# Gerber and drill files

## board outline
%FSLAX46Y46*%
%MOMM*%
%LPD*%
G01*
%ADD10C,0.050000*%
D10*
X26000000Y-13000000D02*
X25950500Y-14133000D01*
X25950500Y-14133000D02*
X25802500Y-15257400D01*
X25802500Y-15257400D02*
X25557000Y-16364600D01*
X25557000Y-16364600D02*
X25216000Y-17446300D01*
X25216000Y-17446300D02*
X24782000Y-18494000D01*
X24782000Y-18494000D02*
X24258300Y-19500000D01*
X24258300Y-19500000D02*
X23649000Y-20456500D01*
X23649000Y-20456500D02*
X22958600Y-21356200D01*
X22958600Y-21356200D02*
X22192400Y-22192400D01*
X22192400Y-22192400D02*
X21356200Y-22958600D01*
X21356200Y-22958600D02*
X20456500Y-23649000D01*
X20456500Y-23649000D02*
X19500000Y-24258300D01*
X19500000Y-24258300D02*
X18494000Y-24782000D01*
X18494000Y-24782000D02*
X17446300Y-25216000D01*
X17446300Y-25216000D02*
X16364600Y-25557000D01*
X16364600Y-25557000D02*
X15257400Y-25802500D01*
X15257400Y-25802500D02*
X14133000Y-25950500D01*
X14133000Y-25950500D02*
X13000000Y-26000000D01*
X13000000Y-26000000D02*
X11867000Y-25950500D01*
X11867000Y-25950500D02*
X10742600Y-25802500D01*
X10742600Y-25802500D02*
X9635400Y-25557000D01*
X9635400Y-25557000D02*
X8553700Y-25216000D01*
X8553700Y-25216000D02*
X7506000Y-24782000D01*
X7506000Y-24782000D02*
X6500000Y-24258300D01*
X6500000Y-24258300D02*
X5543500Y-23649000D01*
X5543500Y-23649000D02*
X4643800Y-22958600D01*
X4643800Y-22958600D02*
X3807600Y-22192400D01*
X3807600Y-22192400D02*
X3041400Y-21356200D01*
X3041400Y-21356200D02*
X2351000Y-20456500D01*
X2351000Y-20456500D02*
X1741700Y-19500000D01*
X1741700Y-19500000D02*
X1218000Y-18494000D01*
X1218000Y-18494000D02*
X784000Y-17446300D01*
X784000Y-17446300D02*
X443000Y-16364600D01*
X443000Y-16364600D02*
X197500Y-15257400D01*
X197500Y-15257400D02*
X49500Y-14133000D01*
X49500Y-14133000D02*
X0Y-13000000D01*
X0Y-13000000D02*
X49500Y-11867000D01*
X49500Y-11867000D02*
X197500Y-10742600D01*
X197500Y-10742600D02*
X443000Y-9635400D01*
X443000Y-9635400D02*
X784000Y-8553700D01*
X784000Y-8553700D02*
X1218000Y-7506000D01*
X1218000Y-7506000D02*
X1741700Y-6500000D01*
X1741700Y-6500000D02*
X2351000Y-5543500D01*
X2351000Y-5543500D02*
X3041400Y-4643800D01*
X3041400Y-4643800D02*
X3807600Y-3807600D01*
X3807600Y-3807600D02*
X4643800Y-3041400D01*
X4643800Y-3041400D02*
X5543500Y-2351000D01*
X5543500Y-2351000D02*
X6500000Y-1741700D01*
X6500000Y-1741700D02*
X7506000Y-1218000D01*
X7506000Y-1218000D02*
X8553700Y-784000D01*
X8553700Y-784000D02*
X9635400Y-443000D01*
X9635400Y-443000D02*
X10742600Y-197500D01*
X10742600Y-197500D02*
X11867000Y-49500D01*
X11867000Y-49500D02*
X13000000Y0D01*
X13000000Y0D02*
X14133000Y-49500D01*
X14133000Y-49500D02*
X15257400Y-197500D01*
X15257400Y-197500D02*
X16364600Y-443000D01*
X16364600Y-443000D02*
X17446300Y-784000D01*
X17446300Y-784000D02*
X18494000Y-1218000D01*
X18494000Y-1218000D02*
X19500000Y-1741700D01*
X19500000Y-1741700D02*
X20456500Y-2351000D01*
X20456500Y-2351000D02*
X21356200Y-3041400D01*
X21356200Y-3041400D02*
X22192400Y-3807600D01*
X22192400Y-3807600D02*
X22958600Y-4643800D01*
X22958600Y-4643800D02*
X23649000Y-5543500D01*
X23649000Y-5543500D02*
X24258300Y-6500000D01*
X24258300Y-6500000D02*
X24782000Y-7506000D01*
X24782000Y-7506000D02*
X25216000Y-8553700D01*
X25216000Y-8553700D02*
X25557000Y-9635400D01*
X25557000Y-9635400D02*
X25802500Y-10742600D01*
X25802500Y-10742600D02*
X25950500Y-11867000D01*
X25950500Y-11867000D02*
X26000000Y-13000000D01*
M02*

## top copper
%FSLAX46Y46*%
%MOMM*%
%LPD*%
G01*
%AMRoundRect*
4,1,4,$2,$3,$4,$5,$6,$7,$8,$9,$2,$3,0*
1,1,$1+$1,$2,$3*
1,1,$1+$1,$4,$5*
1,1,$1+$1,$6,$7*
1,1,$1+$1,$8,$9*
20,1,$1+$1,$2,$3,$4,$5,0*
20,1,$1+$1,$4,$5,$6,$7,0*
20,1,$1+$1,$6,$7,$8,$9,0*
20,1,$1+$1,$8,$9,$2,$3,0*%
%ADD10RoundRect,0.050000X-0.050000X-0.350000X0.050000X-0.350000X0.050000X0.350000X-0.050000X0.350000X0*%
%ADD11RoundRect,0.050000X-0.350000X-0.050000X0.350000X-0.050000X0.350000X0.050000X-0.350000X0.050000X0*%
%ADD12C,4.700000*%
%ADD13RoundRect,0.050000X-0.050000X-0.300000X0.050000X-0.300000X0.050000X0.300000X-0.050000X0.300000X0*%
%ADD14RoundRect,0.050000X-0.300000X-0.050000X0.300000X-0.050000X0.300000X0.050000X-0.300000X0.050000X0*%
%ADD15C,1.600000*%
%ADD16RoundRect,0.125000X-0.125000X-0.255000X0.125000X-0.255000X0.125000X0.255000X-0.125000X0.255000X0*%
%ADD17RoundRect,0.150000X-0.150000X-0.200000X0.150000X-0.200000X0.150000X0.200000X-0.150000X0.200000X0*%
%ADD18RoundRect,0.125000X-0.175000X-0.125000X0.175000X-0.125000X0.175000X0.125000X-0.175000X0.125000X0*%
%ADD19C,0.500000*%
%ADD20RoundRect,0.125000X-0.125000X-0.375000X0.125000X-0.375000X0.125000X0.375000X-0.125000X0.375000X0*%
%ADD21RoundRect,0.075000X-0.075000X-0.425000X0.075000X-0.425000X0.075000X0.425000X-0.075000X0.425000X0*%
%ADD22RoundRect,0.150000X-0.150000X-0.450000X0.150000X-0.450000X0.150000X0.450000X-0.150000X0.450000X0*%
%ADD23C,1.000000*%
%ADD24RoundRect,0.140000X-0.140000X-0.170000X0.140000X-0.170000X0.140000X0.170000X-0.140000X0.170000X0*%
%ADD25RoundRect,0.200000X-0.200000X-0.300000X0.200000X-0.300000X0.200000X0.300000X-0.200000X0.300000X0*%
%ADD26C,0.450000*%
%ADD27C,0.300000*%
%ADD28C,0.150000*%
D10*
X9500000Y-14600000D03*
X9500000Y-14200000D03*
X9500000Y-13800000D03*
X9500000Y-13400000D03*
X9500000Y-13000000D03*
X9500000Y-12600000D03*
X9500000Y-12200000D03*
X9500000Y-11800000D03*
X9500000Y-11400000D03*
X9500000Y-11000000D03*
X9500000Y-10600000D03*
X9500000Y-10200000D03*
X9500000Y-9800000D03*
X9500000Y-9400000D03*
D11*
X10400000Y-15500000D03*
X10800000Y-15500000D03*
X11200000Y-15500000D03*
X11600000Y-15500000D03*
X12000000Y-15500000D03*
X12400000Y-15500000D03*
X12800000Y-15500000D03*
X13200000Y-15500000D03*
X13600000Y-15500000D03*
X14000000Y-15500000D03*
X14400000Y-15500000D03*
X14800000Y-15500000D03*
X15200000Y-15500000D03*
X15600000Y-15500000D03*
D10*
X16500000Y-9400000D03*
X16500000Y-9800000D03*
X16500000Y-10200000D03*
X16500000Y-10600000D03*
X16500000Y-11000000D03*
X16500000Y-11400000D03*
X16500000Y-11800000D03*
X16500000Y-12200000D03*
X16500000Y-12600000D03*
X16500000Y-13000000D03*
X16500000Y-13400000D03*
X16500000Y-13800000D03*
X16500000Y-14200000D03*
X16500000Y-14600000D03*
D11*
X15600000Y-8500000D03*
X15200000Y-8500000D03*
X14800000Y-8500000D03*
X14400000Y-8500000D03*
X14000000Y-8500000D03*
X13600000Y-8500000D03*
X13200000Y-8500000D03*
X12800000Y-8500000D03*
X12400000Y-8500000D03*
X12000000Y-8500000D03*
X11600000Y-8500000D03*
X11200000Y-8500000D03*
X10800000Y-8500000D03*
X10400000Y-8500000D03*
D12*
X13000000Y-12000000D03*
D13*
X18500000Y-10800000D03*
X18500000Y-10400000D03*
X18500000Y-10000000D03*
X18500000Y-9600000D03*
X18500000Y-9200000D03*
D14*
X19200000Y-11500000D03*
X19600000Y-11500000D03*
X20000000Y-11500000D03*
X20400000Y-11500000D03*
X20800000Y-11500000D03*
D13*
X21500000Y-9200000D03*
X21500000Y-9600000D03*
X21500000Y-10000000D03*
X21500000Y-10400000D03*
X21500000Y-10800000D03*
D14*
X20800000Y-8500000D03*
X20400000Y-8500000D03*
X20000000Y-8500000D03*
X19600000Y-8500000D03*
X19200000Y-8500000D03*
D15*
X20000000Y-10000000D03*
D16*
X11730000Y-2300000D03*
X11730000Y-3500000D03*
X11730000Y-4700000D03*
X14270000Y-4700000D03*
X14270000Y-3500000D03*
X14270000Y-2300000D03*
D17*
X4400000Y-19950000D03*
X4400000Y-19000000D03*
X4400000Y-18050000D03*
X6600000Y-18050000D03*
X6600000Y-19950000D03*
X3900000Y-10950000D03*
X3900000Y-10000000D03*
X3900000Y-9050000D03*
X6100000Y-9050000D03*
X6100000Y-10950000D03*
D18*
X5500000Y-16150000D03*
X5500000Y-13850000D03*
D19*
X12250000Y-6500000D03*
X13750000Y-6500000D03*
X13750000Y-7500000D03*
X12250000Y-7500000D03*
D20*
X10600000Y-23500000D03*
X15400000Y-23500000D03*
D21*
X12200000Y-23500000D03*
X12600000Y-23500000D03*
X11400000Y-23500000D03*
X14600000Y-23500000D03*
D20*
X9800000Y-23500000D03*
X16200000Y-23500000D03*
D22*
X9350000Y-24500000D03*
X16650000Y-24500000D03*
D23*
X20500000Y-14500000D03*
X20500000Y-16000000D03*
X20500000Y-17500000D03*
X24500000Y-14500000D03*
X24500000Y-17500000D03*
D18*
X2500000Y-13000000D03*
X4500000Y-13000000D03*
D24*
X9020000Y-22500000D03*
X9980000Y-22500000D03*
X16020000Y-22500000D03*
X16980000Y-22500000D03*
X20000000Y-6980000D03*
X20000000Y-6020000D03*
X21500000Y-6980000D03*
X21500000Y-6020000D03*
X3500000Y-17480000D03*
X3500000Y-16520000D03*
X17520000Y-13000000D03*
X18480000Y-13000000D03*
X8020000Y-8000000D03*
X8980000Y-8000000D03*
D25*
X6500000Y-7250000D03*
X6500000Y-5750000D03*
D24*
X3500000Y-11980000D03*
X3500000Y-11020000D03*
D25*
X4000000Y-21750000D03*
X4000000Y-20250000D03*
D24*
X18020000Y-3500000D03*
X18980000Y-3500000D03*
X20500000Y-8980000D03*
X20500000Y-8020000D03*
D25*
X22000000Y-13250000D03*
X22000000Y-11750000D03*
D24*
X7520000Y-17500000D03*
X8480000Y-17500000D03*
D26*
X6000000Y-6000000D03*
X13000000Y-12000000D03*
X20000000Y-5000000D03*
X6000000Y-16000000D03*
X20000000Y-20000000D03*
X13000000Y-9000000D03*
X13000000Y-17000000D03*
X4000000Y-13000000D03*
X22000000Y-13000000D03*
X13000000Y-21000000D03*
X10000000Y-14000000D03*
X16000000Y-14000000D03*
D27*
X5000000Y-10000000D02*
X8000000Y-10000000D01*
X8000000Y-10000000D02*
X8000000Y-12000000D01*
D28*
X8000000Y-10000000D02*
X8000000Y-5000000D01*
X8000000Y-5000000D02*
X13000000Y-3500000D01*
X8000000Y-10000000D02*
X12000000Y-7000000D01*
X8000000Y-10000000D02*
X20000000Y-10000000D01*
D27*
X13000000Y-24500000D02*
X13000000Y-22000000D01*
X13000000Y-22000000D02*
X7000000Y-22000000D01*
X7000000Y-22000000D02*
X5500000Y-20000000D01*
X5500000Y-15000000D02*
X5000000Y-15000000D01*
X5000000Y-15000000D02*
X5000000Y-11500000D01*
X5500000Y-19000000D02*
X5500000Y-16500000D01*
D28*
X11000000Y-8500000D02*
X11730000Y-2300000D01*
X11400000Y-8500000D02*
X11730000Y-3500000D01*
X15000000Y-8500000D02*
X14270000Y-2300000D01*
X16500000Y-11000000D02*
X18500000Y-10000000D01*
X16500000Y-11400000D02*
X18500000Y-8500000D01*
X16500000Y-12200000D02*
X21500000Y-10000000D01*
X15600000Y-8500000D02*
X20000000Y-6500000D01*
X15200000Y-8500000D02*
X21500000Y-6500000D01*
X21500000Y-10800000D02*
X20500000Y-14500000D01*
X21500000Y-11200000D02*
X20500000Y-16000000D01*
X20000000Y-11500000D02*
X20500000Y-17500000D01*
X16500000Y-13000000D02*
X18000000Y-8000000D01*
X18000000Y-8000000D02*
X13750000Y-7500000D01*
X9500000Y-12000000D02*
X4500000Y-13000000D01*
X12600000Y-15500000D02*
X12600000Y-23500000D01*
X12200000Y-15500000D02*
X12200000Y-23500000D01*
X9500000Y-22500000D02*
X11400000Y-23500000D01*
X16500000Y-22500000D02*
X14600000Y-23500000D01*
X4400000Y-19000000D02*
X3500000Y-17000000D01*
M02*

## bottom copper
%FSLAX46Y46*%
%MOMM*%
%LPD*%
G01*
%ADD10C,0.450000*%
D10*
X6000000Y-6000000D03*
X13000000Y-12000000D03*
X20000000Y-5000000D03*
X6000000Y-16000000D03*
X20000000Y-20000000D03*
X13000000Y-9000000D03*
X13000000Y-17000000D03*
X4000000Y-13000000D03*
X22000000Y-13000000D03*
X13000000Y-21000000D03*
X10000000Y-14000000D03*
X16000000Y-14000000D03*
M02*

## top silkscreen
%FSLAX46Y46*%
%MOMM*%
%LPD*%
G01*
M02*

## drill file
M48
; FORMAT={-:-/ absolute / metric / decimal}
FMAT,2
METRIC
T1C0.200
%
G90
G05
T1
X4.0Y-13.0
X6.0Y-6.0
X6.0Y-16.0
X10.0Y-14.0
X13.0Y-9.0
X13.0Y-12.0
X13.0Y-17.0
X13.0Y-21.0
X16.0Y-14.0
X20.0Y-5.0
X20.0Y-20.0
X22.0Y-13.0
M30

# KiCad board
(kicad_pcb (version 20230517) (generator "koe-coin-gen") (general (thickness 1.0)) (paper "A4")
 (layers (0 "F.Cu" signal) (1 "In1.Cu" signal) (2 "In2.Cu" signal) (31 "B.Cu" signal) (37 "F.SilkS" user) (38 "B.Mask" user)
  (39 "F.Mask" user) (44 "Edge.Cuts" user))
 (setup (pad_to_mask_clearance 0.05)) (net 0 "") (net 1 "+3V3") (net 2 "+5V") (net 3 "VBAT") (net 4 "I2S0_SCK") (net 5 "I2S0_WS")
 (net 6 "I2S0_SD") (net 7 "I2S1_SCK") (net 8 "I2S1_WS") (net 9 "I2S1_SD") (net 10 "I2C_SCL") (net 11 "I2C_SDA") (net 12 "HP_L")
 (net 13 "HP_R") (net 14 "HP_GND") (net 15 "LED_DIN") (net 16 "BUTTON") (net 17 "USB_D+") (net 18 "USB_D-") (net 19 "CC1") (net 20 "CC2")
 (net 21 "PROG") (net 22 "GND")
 (gr_line (start 26.0000 13.0000) (end 25.9505 14.1330) (layer "Edge.Cuts") (width 0.05))
 (gr_line (start 25.9505 14.1330) (end 25.8025 15.2574) (layer "Edge.Cuts") (width 0.05))
 (gr_line (start 25.8025 15.2574) (end 25.5570 16.3646) (layer "Edge.Cuts") (width 0.05))
 (gr_line (start 25.5570 16.3646) (end 25.2160 17.4463) (layer "Edge.Cuts") (width 0.05))
 (gr_line (start 25.2160 17.4463) (end 24.7820 18.4940) (layer "Edge.Cuts") (width 0.05))
 (gr_line (start 24.7820 18.4940) (end 24.2583 19.5000) (layer "Edge.Cuts") (width 0.05))
 (gr_line (start 24.2583 19.5000) (end 23.6490 20.4565) (layer "Edge.Cuts") (width 0.05))
 (gr_line (start 23.6490 20.4565) (end 22.9586 21.3562) (layer "Edge.Cuts") (width 0.05))
 (gr_line (start 22.9586 21.3562) (end 22.1924 22.1924) (layer "Edge.Cuts") (width 0.05))
 (gr_line (start 22.1924 22.1924) (end 21.3562 22.9586) (layer "Edge.Cuts") (width 0.05))
 (gr_line (start 21.3562 22.9586) (end 20.4565 23.6490) (layer "Edge.Cuts") (width 0.05))
 (gr_line (start 20.4565 23.6490) (end 19.5000 24.2583) (layer "Edge.Cuts") (width 0.05))
 (gr_line (start 19.5000 24.2583) (end 18.4940 24.7820) (layer "Edge.Cuts") (width 0.05))
 (gr_line (start 18.4940 24.7820) (end 17.4463 25.2160) (layer "Edge.Cuts") (width 0.05))
 (gr_line (start 17.4463 25.2160) (end 16.3646 25.5570) (layer "Edge.Cuts") (width 0.05))
 (gr_line (start 16.3646 25.5570) (end 15.2574 25.8025) (layer "Edge.Cuts") (width 0.05))
 (gr_line (start 15.2574 25.8025) (end 14.1330 25.9505) (layer "Edge.Cuts") (width 0.05))
 (gr_line (start 14.1330 25.9505) (end 13.0000 26.0000) (layer "Edge.Cuts") (width 0.05))
 (gr_line (start 13.0000 26.0000) (end 11.8670 25.9505) (layer "Edge.Cuts") (width 0.05))
 (gr_line (start 11.8670 25.9505) (end 10.7426 25.8025) (layer "Edge.Cuts") (width 0.05))
 (gr_line (start 10.7426 25.8025) (end 9.6354 25.5570) (layer "Edge.Cuts") (width 0.05))
 (gr_line (start 9.6354 25.5570) (end 8.5537 25.2160) (layer "Edge.Cuts") (width 0.05))
 (gr_line (start 8.5537 25.2160) (end 7.5060 24.7820) (layer "Edge.Cuts") (width 0.05))
 (gr_line (start 7.5060 24.7820) (end 6.5000 24.2583) (layer "Edge.Cuts") (width 0.05))
 (gr_line (start 6.5000 24.2583) (end 5.5435 23.6490) (layer "Edge.Cuts") (width 0.05))
 (gr_line (start 5.5435 23.6490) (end 4.6438 22.9586) (layer "Edge.Cuts") (width 0.05))
 (gr_line (start 4.6438 22.9586) (end 3.8076 22.1924) (layer "Edge.Cuts") (width 0.05))
 (gr_line (start 3.8076 22.1924) (end 3.0414 21.3562) (layer "Edge.Cuts") (width 0.05))
 (gr_line (start 3.0414 21.3562) (end 2.3510 20.4565) (layer "Edge.Cuts") (width 0.05))
 (gr_line (start 2.3510 20.4565) (end 1.7417 19.5000) (layer "Edge.Cuts") (width 0.05))
 (gr_line (start 1.7417 19.5000) (end 1.2180 18.4940) (layer "Edge.Cuts") (width 0.05))
 (gr_line (start 1.2180 18.4940) (end 0.7840 17.4463) (layer "Edge.Cuts") (width 0.05))
 (gr_line (start 0.7840 17.4463) (end 0.4430 16.3646) (layer "Edge.Cuts") (width 0.05))
 (gr_line (start 0.4430 16.3646) (end 0.1975 15.2574) (layer "Edge.Cuts") (width 0.05))
 (gr_line (start 0.1975 15.2574) (end 0.0495 14.1330) (layer "Edge.Cuts") (width 0.05))
 (gr_line (start 0.0495 14.1330) (end 0.0000 13.0000) (layer "Edge.Cuts") (width 0.05))
 (gr_line (start 0.0000 13.0000) (end 0.0495 11.8670) (layer "Edge.Cuts") (width 0.05))
 (gr_line (start 0.0495 11.8670) (end 0.1975 10.7426) (layer "Edge.Cuts") (width 0.05))
 (gr_line (start 0.1975 10.7426) (end 0.4430 9.6354) (layer "Edge.Cuts") (width 0.05))
 (gr_line (start 0.4430 9.6354) (end 0.7840 8.5537) (layer "Edge.Cuts") (width 0.05))
 (gr_line (start 0.7840 8.5537) (end 1.2180 7.5060) (layer "Edge.Cuts") (width 0.05))
 (gr_line (start 1.2180 7.5060) (end 1.7417 6.5000) (layer "Edge.Cuts") (width 0.05))
 (gr_line (start 1.7417 6.5000) (end 2.3510 5.5435) (layer "Edge.Cuts") (width 0.05))
 (gr_line (start 2.3510 5.5435) (end 3.0414 4.6438) (layer "Edge.Cuts") (width 0.05))
 (gr_line (start 3.0414 4.6438) (end 3.8076 3.8076) (layer "Edge.Cuts") (width 0.05))
 (gr_line (start 3.8076 3.8076) (end 4.6438 3.0414) (layer "Edge.Cuts") (width 0.05))
 (gr_line (start 4.6438 3.0414) (end 5.5435 2.3510) (layer "Edge.Cuts") (width 0.05))
 (gr_line (start 5.5435 2.3510) (end 6.5000 1.7417) (layer "Edge.Cuts") (width 0.05))
 (gr_line (start 6.5000 1.7417) (end 7.5060 1.2180) (layer "Edge.Cuts") (width 0.05))
 (gr_line (start 7.5060 1.2180) (end 8.5537 0.7840) (layer "Edge.Cuts") (width 0.05))
 (gr_line (start 8.5537 0.7840) (end 9.6354 0.4430) (layer "Edge.Cuts") (width 0.05))
 (gr_line (start 9.6354 0.4430) (end 10.7426 0.1975) (layer "Edge.Cuts") (width 0.05))
 (gr_line (start 10.7426 0.1975) (end 11.8670 0.0495) (layer "Edge.Cuts") (width 0.05))
 (gr_line (start 11.8670 0.0495) (end 13.0000 0.0000) (layer "Edge.Cuts") (width 0.05))
 (gr_line (start 13.0000 0.0000) (end 14.1330 0.0495) (layer "Edge.Cuts") (width 0.05))
 (gr_line (start 14.1330 0.0495) (end 15.2574 0.1975) (layer "Edge.Cuts") (width 0.05))
 (gr_line (start 15.2574 0.1975) (end 16.3646 0.4430) (layer "Edge.Cuts") (width 0.05))
 (gr_line (start 16.3646 0.4430) (end 17.4463 0.7840) (layer "Edge.Cuts") (width 0.05))
 (gr_line (start 17.4463 0.7840) (end 18.4940 1.2180) (layer "Edge.Cuts") (width 0.05))
 (gr_line (start 18.4940 1.2180) (end 19.5000 1.7417) (layer "Edge.Cuts") (width 0.05))
 (gr_line (start 19.5000 1.7417) (end 20.4565 2.3510) (layer "Edge.Cuts") (width 0.05))
 (gr_line (start 20.4565 2.3510) (end 21.3562 3.0414) (layer "Edge.Cuts") (width 0.05))
 (gr_line (start 21.3562 3.0414) (end 22.1924 3.8076) (layer "Edge.Cuts") (width 0.05))
 (gr_line (start 22.1924 3.8076) (end 22.9586 4.6438) (layer "Edge.Cuts") (width 0.05))
 (gr_line (start 22.9586 4.6438) (end 23.6490 5.5435) (layer "Edge.Cuts") (width 0.05))
 (gr_line (start 23.6490 5.5435) (end 24.2583 6.5000) (layer "Edge.Cuts") (width 0.05))
 (gr_line (start 24.2583 6.5000) (end 24.7820 7.5060) (layer "Edge.Cuts") (width 0.05))
 (gr_line (start 24.7820 7.5060) (end 25.2160 8.5537) (layer "Edge.Cuts") (width 0.05))
 (gr_line (start 25.2160 8.5537) (end 25.5570 9.6354) (layer "Edge.Cuts") (width 0.05))
 (gr_line (start 25.5570 9.6354) (end 25.8025 10.7426) (layer "Edge.Cuts") (width 0.05))
 (gr_line (start 25.8025 10.7426) (end 25.9505 11.8670) (layer "Edge.Cuts") (width 0.05))
 (gr_line (start 25.9505 11.8670) (end 26.0000 13.0000) (layer "Edge.Cuts") (width 0.05))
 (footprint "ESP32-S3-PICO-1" (at 13.0 12.0 0) (layer "F.Cu") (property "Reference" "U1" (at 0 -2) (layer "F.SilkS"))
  (pad "1" smd roundrect (at -3.5 2.6) (size 0.2 0.8) (layers "F.Cu" "F.Paste" "F.Mask") (roundrect_rratio 0.25))
  (pad "2" smd roundrect (at -3.5 2.2) (size 0.2 0.8) (layers "F.Cu" "F.Paste" "F.Mask") (roundrect_rratio 0.25))
  (pad "3" smd roundrect (at -3.5 1.8) (size 0.2 0.8) (layers "F.Cu" "F.Paste" "F.Mask") (roundrect_rratio 0.25))
  (pad "4" smd roundrect (at -3.5 1.4) (size 0.2 0.8) (layers "F.Cu" "F.Paste" "F.Mask") (roundrect_rratio 0.25))
  (pad "5" smd roundrect (at -3.5 1.0) (size 0.2 0.8) (layers "F.Cu" "F.Paste" "F.Mask") (roundrect_rratio 0.25))
  (pad "6" smd roundrect (at -3.5 0.6000000000000001) (size 0.2 0.8) (layers "F.Cu" "F.Paste" "F.Mask") (roundrect_rratio 0.25))
  (pad "7" smd roundrect (at -3.5 0.19999999999999973) (size 0.2 0.8) (layers "F.Cu" "F.Paste" "F.Mask") (roundrect_rratio 0.25))
  (pad "8" smd roundrect (at -3.5 -0.20000000000000018) (size 0.2 0.8) (layers "F.Cu" "F.Paste" "F.Mask") (roundrect_rratio 0.25))
  (pad "9" smd roundrect (at -3.5 -0.6000000000000001) (size 0.2 0.8) (layers "F.Cu" "F.Paste" "F.Mask") (roundrect_rratio 0.25))
  (pad "10" smd roundrect (at -3.5 -1.0) (size 0.2 0.8) (layers "F.Cu" "F.Paste" "F.Mask") (roundrect_rratio 0.25))
  (pad "11" smd roundrect (at -3.5 -1.4) (size 0.2 0.8) (layers "F.Cu" "F.Paste" "F.Mask") (roundrect_rratio 0.25))
  (pad "12" smd roundrect (at -3.5 -1.8000000000000003) (size 0.2 0.8) (layers "F.Cu" "F.Paste" "F.Mask") (roundrect_rratio 0.25))
  (pad "13" smd roundrect (at -3.5 -2.2000000000000006) (size 0.2 0.8) (layers "F.Cu" "F.Paste" "F.Mask") (roundrect_rratio 0.25))
  (pad "14" smd roundrect (at -3.5 -2.6) (size 0.2 0.8) (layers "F.Cu" "F.Paste" "F.Mask") (roundrect_rratio 0.25))
  (pad "15" smd roundrect (at -2.6 3.5) (size 0.8 0.2) (layers "F.Cu" "F.Paste" "F.Mask") (roundrect_rratio 0.25))
  (pad "16" smd roundrect (at -2.2 3.5) (size 0.8 0.2) (layers "F.Cu" "F.Paste" "F.Mask") (roundrect_rratio 0.25))
  (pad "17" smd roundrect (at -1.8 3.5) (size 0.8 0.2) (layers "F.Cu" "F.Paste" "F.Mask") (roundrect_rratio 0.25))
  (pad "18" smd roundrect (at -1.4 3.5) (size 0.8 0.2) (layers "F.Cu" "F.Paste" "F.Mask") (roundrect_rratio 0.25))
  (pad "19" smd roundrect (at -1.0 3.5) (size 0.8 0.2) (layers "F.Cu" "F.Paste" "F.Mask") (roundrect_rratio 0.25))
  (pad "20" smd roundrect (at -0.6000000000000001 3.5) (size 0.8 0.2) (layers "F.Cu" "F.Paste" "F.Mask") (roundrect_rratio 0.25))
  (pad "21" smd roundrect (at -0.19999999999999973 3.5) (size 0.8 0.2) (layers "F.Cu" "F.Paste" "F.Mask") (roundrect_rratio 0.25))
  (pad "22" smd roundrect (at 0.20000000000000018 3.5) (size 0.8 0.2) (layers "F.Cu" "F.Paste" "F.Mask") (roundrect_rratio 0.25))
  (pad "23" smd roundrect (at 0.6000000000000001 3.5) (size 0.8 0.2) (layers "F.Cu" "F.Paste" "F.Mask") (roundrect_rratio 0.25))
  (pad "24" smd roundrect (at 1.0 3.5) (size 0.8 0.2) (layers "F.Cu" "F.Paste" "F.Mask") (roundrect_rratio 0.25))
  (pad "25" smd roundrect (at 1.4 3.5) (size 0.8 0.2) (layers "F.Cu" "F.Paste" "F.Mask") (roundrect_rratio 0.25))
  (pad "26" smd roundrect (at 1.8000000000000003 3.5) (size 0.8 0.2) (layers "F.Cu" "F.Paste" "F.Mask") (roundrect_rratio 0.25))
  (pad "27" smd roundrect (at 2.2000000000000006 3.5) (size 0.8 0.2) (layers "F.Cu" "F.Paste" "F.Mask") (roundrect_rratio 0.25))
  (pad "28" smd roundrect (at 2.6 3.5) (size 0.8 0.2) (layers "F.Cu" "F.Paste" "F.Mask") (roundrect_rratio 0.25))
  (pad "29" smd roundrect (at 3.5 -2.6) (size 0.2 0.8) (layers "F.Cu" "F.Paste" "F.Mask") (roundrect_rratio 0.25))
  (pad "30" smd roundrect (at 3.5 -2.2) (size 0.2 0.8) (layers "F.Cu" "F.Paste" "F.Mask") (roundrect_rratio 0.25))
  (pad "31" smd roundrect (at 3.5 -1.8) (size 0.2 0.8) (layers "F.Cu" "F.Paste" "F.Mask") (roundrect_rratio 0.25))
  (pad "32" smd roundrect (at 3.5 -1.4) (size 0.2 0.8) (layers "F.Cu" "F.Paste" "F.Mask") (roundrect_rratio 0.25))
  (pad "33" smd roundrect (at 3.5 -1.0) (size 0.2 0.8) (layers "F.Cu" "F.Paste" "F.Mask") (roundrect_rratio 0.25))
  (pad "34" smd roundrect (at 3.5 -0.6000000000000001) (size 0.2 0.8) (layers "F.Cu" "F.Paste" "F.Mask") (roundrect_rratio 0.25))
  (pad "35" smd roundrect (at 3.5 -0.19999999999999973) (size 0.2 0.8) (layers "F.Cu" "F.Paste" "F.Mask") (roundrect_rratio 0.25))
  (pad "36" smd roundrect (at 3.5 0.20000000000000018) (size 0.2 0.8) (layers "F.Cu" "F.Paste" "F.Mask") (roundrect_rratio 0.25))
  (pad "37" smd roundrect (at 3.5 0.6000000000000001) (size 0.2 0.8) (layers "F.Cu" "F.Paste" "F.Mask") (roundrect_rratio 0.25))
  (pad "38" smd roundrect (at 3.5 1.0) (size 0.2 0.8) (layers "F.Cu" "F.Paste" "F.Mask") (roundrect_rratio 0.25))
  (pad "39" smd roundrect (at 3.5 1.4) (size 0.2 0.8) (layers "F.Cu" "F.Paste" "F.Mask") (roundrect_rratio 0.25))
  (pad "40" smd roundrect (at 3.5 1.8000000000000003) (size 0.2 0.8) (layers "F.Cu" "F.Paste" "F.Mask") (roundrect_rratio 0.25))
  (pad "41" smd roundrect (at 3.5 2.2000000000000006) (size 0.2 0.8) (layers "F.Cu" "F.Paste" "F.Mask") (roundrect_rratio 0.25))
  (pad "42" smd roundrect (at 3.5 2.6) (size 0.2 0.8) (layers "F.Cu" "F.Paste" "F.Mask") (roundrect_rratio 0.25))
  (pad "43" smd roundrect (at 2.6 -3.5) (size 0.8 0.2) (layers "F.Cu" "F.Paste" "F.Mask") (roundrect_rratio 0.25))
  (pad "44" smd roundrect (at 2.2 -3.5) (size 0.8 0.2) (layers "F.Cu" "F.Paste" "F.Mask") (roundrect_rratio 0.25))
  (pad "45" smd roundrect (at 1.8 -3.5) (size 0.8 0.2) (layers "F.Cu" "F.Paste" "F.Mask") (roundrect_rratio 0.25))
  (pad "46" smd roundrect (at 1.4 -3.5) (size 0.8 0.2) (layers "F.Cu" "F.Paste" "F.Mask") (roundrect_rratio 0.25))
  (pad "47" smd roundrect (at 1.0 -3.5) (size 0.8 0.2) (layers "F.Cu" "F.Paste" "F.Mask") (roundrect_rratio 0.25))
  (pad "48" smd roundrect (at 0.6000000000000001 -3.5) (size 0.8 0.2) (layers "F.Cu" "F.Paste" "F.Mask") (roundrect_rratio 0.25))
  (pad "49" smd roundrect (at 0.19999999999999973 -3.5) (size 0.8 0.2) (layers "F.Cu" "F.Paste" "F.Mask") (roundrect_rratio 0.25))
  (pad "50" smd roundrect (at -0.20000000000000018 -3.5) (size 0.8 0.2) (layers "F.Cu" "F.Paste" "F.Mask") (roundrect_rratio 0.25))
  (pad "51" smd roundrect (at -0.6000000000000001 -3.5) (size 0.8 0.2) (layers "F.Cu" "F.Paste" "F.Mask") (roundrect_rratio 0.25))
  (pad "52" smd roundrect (at -1.0 -3.5) (size 0.8 0.2) (layers "F.Cu" "F.Paste" "F.Mask") (roundrect_rratio 0.25))
  (pad "53" smd roundrect (at -1.4 -3.5) (size 0.8 0.2) (layers "F.Cu" "F.Paste" "F.Mask") (roundrect_rratio 0.25))
  (pad "54" smd roundrect (at -1.8000000000000003 -3.5) (size 0.8 0.2) (layers "F.Cu" "F.Paste" "F.Mask") (roundrect_rratio 0.25))
  (pad "55" smd roundrect (at -2.2000000000000006 -3.5) (size 0.8 0.2) (layers "F.Cu" "F.Paste" "F.Mask") (roundrect_rratio 0.25))
  (pad "56" smd roundrect (at -2.6 -3.5) (size 0.8 0.2) (layers "F.Cu" "F.Paste" "F.Mask") (roundrect_rratio 0.25))
  (pad "57" smd circle (at 0.0 0.0) (size 4.7 4.7) (layers "F.Cu" "F.Paste" "F.Mask") (roundrect_rratio 0.25)))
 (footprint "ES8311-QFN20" (at 20.0 10.0 0) (layer "F.Cu") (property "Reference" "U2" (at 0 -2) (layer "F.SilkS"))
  (pad "1" smd roundrect (at -1.5 0.8) (size 0.2 0.7) (layers "F.Cu" "F.Paste" "F.Mask") (roundrect_rratio 0.25))
  (pad "2" smd roundrect (at -1.5 0.4) (size 0.2 0.7) (layers "F.Cu" "F.Paste" "F.Mask") (roundrect_rratio 0.25))
  (pad "3" smd roundrect (at -1.5 0.0) (size 0.2 0.7) (layers "F.Cu" "F.Paste" "F.Mask") (roundrect_rratio 0.25))
  (pad "4" smd roundrect (at -1.5 -0.40000000000000013) (size 0.2 0.7) (layers "F.Cu" "F.Paste" "F.Mask") (roundrect_rratio 0.25))
  (pad "5" smd roundrect (at -1.5 -0.8) (size 0.2 0.7) (layers "F.Cu" "F.Paste" "F.Mask") (roundrect_rratio 0.25))
  (pad "6" smd roundrect (at -0.8 1.5) (size 0.7 0.2) (layers "F.Cu" "F.Paste" "F.Mask") (roundrect_rratio 0.25))
  (pad "7" smd roundrect (at -0.4 1.5) (size 0.7 0.2) (layers "F.Cu" "F.Paste" "F.Mask") (roundrect_rratio 0.25))
  (pad "8" smd roundrect (at 0.0 1.5) (size 0.7 0.2) (layers "F.Cu" "F.Paste" "F.Mask") (roundrect_rratio 0.25))
  (pad "9" smd roundrect (at 0.40000000000000013 1.5) (size 0.7 0.2) (layers "F.Cu" "F.Paste" "F.Mask") (roundrect_rratio 0.25))
  (pad "10" smd roundrect (at 0.8 1.5) (size 0.7 0.2) (layers "F.Cu" "F.Paste" "F.Mask") (roundrect_rratio 0.25))
  (pad "11" smd roundrect (at 1.5 -0.8) (size 0.2 0.7) (layers "F.Cu" "F.Paste" "F.Mask") (roundrect_rratio 0.25))
  (pad "12" smd roundrect (at 1.5 -0.4) (size 0.2 0.7) (layers "F.Cu" "F.Paste" "F.Mask") (roundrect_rratio 0.25))
  (pad "13" smd roundrect (at 1.5 0.0) (size 0.2 0.7) (layers "F.Cu" "F.Paste" "F.Mask") (roundrect_rratio 0.25))
  (pad "14" smd roundrect (at 1.5 0.40000000000000013) (size 0.2 0.7) (layers "F.Cu" "F.Paste" "F.Mask") (roundrect_rratio 0.25))
  (pad "15" smd roundrect (at 1.5 0.8) (size 0.2 0.7) (layers "F.Cu" "F.Paste" "F.Mask") (roundrect_rratio 0.25))
  (pad "16" smd roundrect (at 0.8 -1.5) (size 0.7 0.2) (layers "F.Cu" "F.Paste" "F.Mask") (roundrect_rratio 0.25))
  (pad "17" smd roundrect (at 0.4 -1.5) (size 0.7 0.2) (layers "F.Cu" "F.Paste" "F.Mask") (roundrect_rratio 0.25))
  (pad "18" smd roundrect (at 0.0 -1.5) (size 0.7 0.2) (layers "F.Cu" "F.Paste" "F.Mask") (roundrect_rratio 0.25))
  (pad "19" smd roundrect (at -0.40000000000000013 -1.5) (size 0.7 0.2) (layers "F.Cu" "F.Paste" "F.Mask") (roundrect_rratio 0.25))
  (pad "20" smd roundrect (at -0.8 -1.5) (size 0.7 0.2) (layers "F.Cu" "F.Paste" "F.Mask") (roundrect_rratio 0.25))
  (pad "21" smd circle (at 0.0 0.0) (size 1.6 1.6) (layers "F.Cu" "F.Paste" "F.Mask") (roundrect_rratio 0.25)))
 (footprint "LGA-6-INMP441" (at 13.0 3.5 0) (layer "F.Cu") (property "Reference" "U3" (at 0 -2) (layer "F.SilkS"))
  (pad "1" smd roundrect (at -1.27 -1.2) (size 0.5 0.76) (layers "F.Cu" "F.Paste" "F.Mask") (roundrect_rratio 0.25))
  (pad "2" smd roundrect (at -1.27 0.0) (size 0.5 0.76) (layers "F.Cu" "F.Paste" "F.Mask") (roundrect_rratio 0.25))
  (pad "3" smd roundrect (at -1.27 1.2) (size 0.5 0.76) (layers "F.Cu" "F.Paste" "F.Mask") (roundrect_rratio 0.25))
  (pad "4" smd roundrect (at 1.27 1.2) (size 0.5 0.76) (layers "F.Cu" "F.Paste" "F.Mask") (roundrect_rratio 0.25))
  (pad "5" smd roundrect (at 1.27 0.0) (size 0.5 0.76) (layers "F.Cu" "F.Paste" "F.Mask") (roundrect_rratio 0.25))
  (pad "6" smd roundrect (at 1.27 -1.2) (size 0.5 0.76) (layers "F.Cu" "F.Paste" "F.Mask") (roundrect_rratio 0.25)))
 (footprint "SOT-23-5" (at 5.5 19.0 0) (layer "F.Cu") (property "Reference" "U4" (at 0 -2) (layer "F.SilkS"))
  (pad "1" smd roundrect (at -1.1 0.95) (size 0.6 0.7) (layers "F.Cu" "F.Paste" "F.Mask") (roundrect_rratio 0.25))
  (pad "2" smd roundrect (at -1.1 0.0) (size 0.6 0.7) (layers "F.Cu" "F.Paste" "F.Mask") (roundrect_rratio 0.25))
  (pad "3" smd roundrect (at -1.1 -0.95) (size 0.6 0.7) (layers "F.Cu" "F.Paste" "F.Mask") (roundrect_rratio 0.25))
  (pad "4" smd roundrect (at 1.1 -0.95) (size 0.6 0.7) (layers "F.Cu" "F.Paste" "F.Mask") (roundrect_rratio 0.25))
  (pad "5" smd roundrect (at 1.1 0.95) (size 0.6 0.7) (layers "F.Cu" "F.Paste" "F.Mask") (roundrect_rratio 0.25)))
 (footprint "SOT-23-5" (at 5.0 10.0 0) (layer "F.Cu") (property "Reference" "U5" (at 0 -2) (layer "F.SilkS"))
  (pad "1" smd roundrect (at -1.1 0.95) (size 0.6 0.7) (layers "F.Cu" "F.Paste" "F.Mask") (roundrect_rratio 0.25))
  (pad "2" smd roundrect (at -1.1 0.0) (size 0.6 0.7) (layers "F.Cu" "F.Paste" "F.Mask") (roundrect_rratio 0.25))
  (pad "3" smd roundrect (at -1.1 -0.95) (size 0.6 0.7) (layers "F.Cu" "F.Paste" "F.Mask") (roundrect_rratio 0.25))
  (pad "4" smd roundrect (at 1.1 -0.95) (size 0.6 0.7) (layers "F.Cu" "F.Paste" "F.Mask") (roundrect_rratio 0.25))
  (pad "5" smd roundrect (at 1.1 0.95) (size 0.6 0.7) (layers "F.Cu" "F.Paste" "F.Mask") (roundrect_rratio 0.25)))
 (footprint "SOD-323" (at 5.5 15.0 90) (layer "F.Cu") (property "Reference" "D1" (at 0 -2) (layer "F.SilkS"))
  (pad "1" smd roundrect (at -1.15 0.0) (size 0.6 0.5) (layers "F.Cu" "F.Paste" "F.Mask") (roundrect_rratio 0.25))
  (pad "2" smd roundrect (at 1.15 0.0) (size 0.6 0.5) (layers "F.Cu" "F.Paste" "F.Mask") (roundrect_rratio 0.25)))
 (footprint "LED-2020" (at 13.0 7.0 0) (layer "F.Cu") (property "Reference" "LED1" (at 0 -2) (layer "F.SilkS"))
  (pad "1" smd circle (at -0.75 -0.5) (size 0.5 0.5) (layers "F.Cu" "F.Paste" "F.Mask") (roundrect_rratio 0.25))
  (pad "2" smd circle (at 0.75 -0.5) (size 0.5 0.5) (layers "F.Cu" "F.Paste" "F.Mask") (roundrect_rratio 0.25))
  (pad "3" smd circle (at 0.75 0.5) (size 0.5 0.5) (layers "F.Cu" "F.Paste" "F.Mask") (roundrect_rratio 0.25))
  (pad "4" smd circle (at -0.75 0.5) (size 0.5 0.5) (layers "F.Cu" "F.Paste" "F.Mask") (roundrect_rratio 0.25)))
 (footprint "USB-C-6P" (at 13.0 24.5 0) (layer "F.Cu") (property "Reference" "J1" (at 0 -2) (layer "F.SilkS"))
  (pad "V1" smd roundrect (at -2.4 -1.0) (size 0.5 1.0) (layers "F.Cu" "F.Paste" "F.Mask") (roundrect_rratio 0.25))
  (pad "V2" smd roundrect (at 2.4 -1.0) (size 0.5 1.0) (layers "F.Cu" "F.Paste" "F.Mask") (roundrect_rratio 0.25))
  (pad "D-" smd roundrect (at -0.8 -1.0) (size 0.3 1.0) (layers "F.Cu" "F.Paste" "F.Mask") (roundrect_rratio 0.25))
  (pad "D+" smd roundrect (at -0.4 -1.0) (size 0.3 1.0) (layers "F.Cu" "F.Paste" "F.Mask") (roundrect_rratio 0.25))
  (pad "C1" smd roundrect (at -1.6 -1.0) (size 0.3 1.0) (layers "F.Cu" "F.Paste" "F.Mask") (roundrect_rratio 0.25))
  (pad "C2" smd roundrect (at 1.6 -1.0) (size 0.3 1.0) (layers "F.Cu" "F.Paste" "F.Mask") (roundrect_rratio 0.25))
  (pad "G1" smd roundrect (at -3.2 -1.0) (size 0.5 1.0) (layers "F.Cu" "F.Paste" "F.Mask") (roundrect_rratio 0.25))
  (pad "G2" smd roundrect (at 3.2 -1.0) (size 0.5 1.0) (layers "F.Cu" "F.Paste" "F.Mask") (roundrect_rratio 0.25))
  (pad "S1" smd roundrect (at -3.65 0.0) (size 0.6 1.2) (layers "F.Cu" "F.Paste" "F.Mask") (roundrect_rratio 0.25))
  (pad "S2" smd roundrect (at 3.65 0.0) (size 0.6 1.2) (layers "F.Cu" "F.Paste" "F.Mask") (roundrect_rratio 0.25)))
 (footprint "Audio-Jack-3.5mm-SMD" (at 22.5 16.0 0) (layer "F.Cu") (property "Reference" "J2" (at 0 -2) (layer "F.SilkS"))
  (pad "1" smd circle (at -2.0 -1.5) (size 1.0 1.0) (layers "F.Cu" "F.Paste" "F.Mask") (roundrect_rratio 0.25))
  (pad "2" smd circle (at -2.0 0.0) (size 1.0 1.0) (layers "F.Cu" "F.Paste" "F.Mask") (roundrect_rratio 0.25))
  (pad "3" smd circle (at -2.0 1.5) (size 1.0 1.0) (layers "F.Cu" "F.Paste" "F.Mask") (roundrect_rratio 0.25))
  (pad "4" smd circle (at 2.0 -1.5) (size 1.0 1.0) (layers "F.Cu" "F.Paste" "F.Mask") (roundrect_rratio 0.25))
  (pad "5" smd circle (at 2.0 1.5) (size 1.0 1.0) (layers "F.Cu" "F.Paste" "F.Mask") (roundrect_rratio 0.25)))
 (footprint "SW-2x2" (at 3.5 13.0 0) (layer "F.Cu") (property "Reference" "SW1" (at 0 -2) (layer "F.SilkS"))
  (pad "1" smd roundrect (at -1.0 0.0) (size 0.6 0.5) (layers "F.Cu" "F.Paste" "F.Mask") (roundrect_rratio 0.25))
  (pad "2" smd roundrect (at 1.0 0.0) (size 0.6 0.5) (layers "F.Cu" "F.Paste" "F.Mask") (roundrect_rratio 0.25)))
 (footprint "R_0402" (at 9.5 22.5 0) (layer "F.Cu") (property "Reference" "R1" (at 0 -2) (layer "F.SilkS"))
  (pad "1" smd roundrect (at -0.48 0.0) (size 0.56 0.62) (layers "F.Cu" "F.Paste" "F.Mask") (roundrect_rratio 0.25))
  (pad "2" smd roundrect (at 0.48 0.0) (size 0.56 0.62) (layers "F.Cu" "F.Paste" "F.Mask") (roundrect_rratio 0.25)))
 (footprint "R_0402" (at 16.5 22.5 0) (layer "F.Cu") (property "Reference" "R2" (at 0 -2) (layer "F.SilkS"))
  (pad "1" smd roundrect (at -0.48 0.0) (size 0.56 0.62) (layers "F.Cu" "F.Paste" "F.Mask") (roundrect_rratio 0.25))
  (pad "2" smd roundrect (at 0.48 0.0) (size 0.56 0.62) (layers "F.Cu" "F.Paste" "F.Mask") (roundrect_rratio 0.25)))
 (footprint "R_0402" (at 20.0 6.5 90) (layer "F.Cu") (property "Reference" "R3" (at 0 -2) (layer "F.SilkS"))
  (pad "1" smd roundrect (at -0.48 0.0) (size 0.56 0.62) (layers "F.Cu" "F.Paste" "F.Mask") (roundrect_rratio 0.25))
  (pad "2" smd roundrect (at 0.48 0.0) (size 0.56 0.62) (layers "F.Cu" "F.Paste" "F.Mask") (roundrect_rratio 0.25)))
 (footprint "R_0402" (at 21.5 6.5 90) (layer "F.Cu") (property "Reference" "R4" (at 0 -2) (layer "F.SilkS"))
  (pad "1" smd roundrect (at -0.48 0.0) (size 0.56 0.62) (layers "F.Cu" "F.Paste" "F.Mask") (roundrect_rratio 0.25))
  (pad "2" smd roundrect (at 0.48 0.0) (size 0.56 0.62) (layers "F.Cu" "F.Paste" "F.Mask") (roundrect_rratio 0.25)))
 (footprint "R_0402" (at 3.5 17.0 90) (layer "F.Cu") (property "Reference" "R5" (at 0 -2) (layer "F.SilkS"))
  (pad "1" smd roundrect (at -0.48 0.0) (size 0.56 0.62) (layers "F.Cu" "F.Paste" "F.Mask") (roundrect_rratio 0.25))
  (pad "2" smd roundrect (at 0.48 0.0) (size 0.56 0.62) (layers "F.Cu" "F.Paste" "F.Mask") (roundrect_rratio 0.25)))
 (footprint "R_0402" (at 18.0 13.0 0) (layer "F.Cu") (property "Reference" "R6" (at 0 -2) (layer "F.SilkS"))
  (pad "1" smd roundrect (at -0.48 0.0) (size 0.56 0.62) (layers "F.Cu" "F.Paste" "F.Mask") (roundrect_rratio 0.25))
  (pad "2" smd roundrect (at 0.48 0.0) (size 0.56 0.62) (layers "F.Cu" "F.Paste" "F.Mask") (roundrect_rratio 0.25)))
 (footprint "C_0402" (at 8.5 8.0 0) (layer "F.Cu") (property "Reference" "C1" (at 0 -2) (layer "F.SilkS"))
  (pad "1" smd roundrect (at -0.48 0.0) (size 0.56 0.62) (layers "F.Cu" "F.Paste" "F.Mask") (roundrect_rratio 0.25))
  (pad "2" smd roundrect (at 0.48 0.0) (size 0.56 0.62) (layers "F.Cu" "F.Paste" "F.Mask") (roundrect_rratio 0.25)))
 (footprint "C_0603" (at 6.5 6.5 90) (layer "F.Cu") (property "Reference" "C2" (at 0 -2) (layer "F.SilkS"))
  (pad "1" smd roundrect (at -0.75 0.0) (size 0.8 1.0) (layers "F.Cu" "F.Paste" "F.Mask") (roundrect_rratio 0.25))
  (pad "2" smd roundrect (at 0.75 0.0) (size 0.8 1.0) (layers "F.Cu" "F.Paste" "F.Mask") (roundrect_rratio 0.25)))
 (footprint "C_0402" (at 3.5 11.5 90) (layer "F.Cu") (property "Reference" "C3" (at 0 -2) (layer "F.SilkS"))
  (pad "1" smd roundrect (at -0.48 0.0) (size 0.56 0.62) (layers "F.Cu" "F.Paste" "F.Mask") (roundrect_rratio 0.25))
  (pad "2" smd roundrect (at 0.48 0.0) (size 0.56 0.62) (layers "F.Cu" "F.Paste" "F.Mask") (roundrect_rratio 0.25)))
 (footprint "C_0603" (at 4.0 21.0 90) (layer "F.Cu") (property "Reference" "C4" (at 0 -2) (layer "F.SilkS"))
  (pad "1" smd roundrect (at -0.75 0.0) (size 0.8 1.0) (layers "F.Cu" "F.Paste" "F.Mask") (roundrect_rratio 0.25))
  (pad "2" smd roundrect (at 0.75 0.0) (size 0.8 1.0) (layers "F.Cu" "F.Paste" "F.Mask") (roundrect_rratio 0.25)))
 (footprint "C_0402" (at 18.5 3.5 0) (layer "F.Cu") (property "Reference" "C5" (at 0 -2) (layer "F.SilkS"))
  (pad "1" smd roundrect (at -0.48 0.0) (size 0.56 0.62) (layers "F.Cu" "F.Paste" "F.Mask") (roundrect_rratio 0.25))
  (pad "2" smd roundrect (at 0.48 0.0) (size 0.56 0.62) (layers "F.Cu" "F.Paste" "F.Mask") (roundrect_rratio 0.25)))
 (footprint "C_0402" (at 20.5 8.5 90) (layer "F.Cu") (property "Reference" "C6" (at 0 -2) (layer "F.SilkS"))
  (pad "1" smd roundrect (at -0.48 0.0) (size 0.56 0.62) (layers "F.Cu" "F.Paste" "F.Mask") (roundrect_rratio 0.25))
  (pad "2" smd roundrect (at 0.48 0.0) (size 0.56 0.62) (layers "F.Cu" "F.Paste" "F.Mask") (roundrect_rratio 0.25)))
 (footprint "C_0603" (at 22.0 12.5 90) (layer "F.Cu") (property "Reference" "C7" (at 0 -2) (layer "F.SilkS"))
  (pad "1" smd roundrect (at -0.75 0.0) (size 0.8 1.0) (layers "F.Cu" "F.Paste" "F.Mask") (roundrect_rratio 0.25))
  (pad "2" smd roundrect (at 0.75 0.0) (size 0.8 1.0) (layers "F.Cu" "F.Paste" "F.Mask") (roundrect_rratio 0.25)))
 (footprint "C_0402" (at 8.0 17.5 0) (layer "F.Cu") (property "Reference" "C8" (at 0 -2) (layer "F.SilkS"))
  (pad "1" smd roundrect (at -0.48 0.0) (size 0.56 0.62) (layers "F.Cu" "F.Paste" "F.Mask") (roundrect_rratio 0.25))
  (pad "2" smd roundrect (at 0.48 0.0) (size 0.56 0.62) (layers "F.Cu" "F.Paste" "F.Mask") (roundrect_rratio 0.25)))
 (segment (start 5.0 10.0) (end 8.0 10.0) (width 0.3) (layer "F.Cu") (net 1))
 (segment (start 8.0 10.0) (end 8.0 12.0) (width 0.3) (layer "F.Cu") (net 1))
 (segment (start 8.0 10.0) (end 8.0 5.0) (width 0.15) (layer "F.Cu") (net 1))
 (segment (start 8.0 5.0) (end 13.0 3.5) (width 0.15) (layer "F.Cu") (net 1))
 (segment (start 8.0 10.0) (end 12.0 7.0) (width 0.15) (layer "F.Cu") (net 1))
 (segment (start 8.0 10.0) (end 20.0 10.0) (width 0.15) (layer "F.Cu") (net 1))
 (segment (start 13.0 24.5) (end 13.0 22.0) (width 0.3) (layer "F.Cu") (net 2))
 (segment (start 13.0 22.0) (end 7.0 22.0) (width 0.3) (layer "F.Cu") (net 2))
 (segment (start 7.0 22.0) (end 5.5 20.0) (width 0.3) (layer "F.Cu") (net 2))
 (segment (start 5.5 15.0) (end 5.0 15.0) (width 0.3) (layer "F.Cu") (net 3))
 (segment (start 5.0 15.0) (end 5.0 11.5) (width 0.3) (layer "F.Cu") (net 3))
 (segment (start 5.5 19.0) (end 5.5 16.5) (width 0.3) (layer "F.Cu") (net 3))
 (segment (start 11.0 8.5) (end 11.73 2.3) (width 0.15) (layer "F.Cu") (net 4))
 (segment (start 11.4 8.5) (end 11.73 3.5) (width 0.15) (layer "F.Cu") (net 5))
 (segment (start 15.0 8.5) (end 14.27 2.3) (width 0.15) (layer "F.Cu") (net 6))
 (segment (start 16.5 11.0) (end 18.5 10.0) (width 0.15) (layer "F.Cu") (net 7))
 (segment (start 16.5 11.4) (end 18.5 8.5) (width 0.15) (layer "F.Cu") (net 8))
 (segment (start 16.5 12.2) (end 21.5 10.0) (width 0.15) (layer "F.Cu") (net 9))
 (segment (start 15.6 8.5) (end 20.0 6.5) (width 0.15) (layer "F.Cu") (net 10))
 (segment (start 15.2 8.5) (end 21.5 6.5) (width 0.15) (layer "F.Cu") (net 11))
 (segment (start 21.5 10.8) (end 20.5 14.5) (width 0.15) (layer "F.Cu") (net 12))
 (segment (start 21.5 11.2) (end 20.5 16.0) (width 0.15) (layer "F.Cu") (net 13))
 (segment (start 20.0 11.5) (end 20.5 17.5) (width 0.15) (layer "F.Cu") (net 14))
 (segment (start 16.5 13.0) (end 18.0 8.0) (width 0.15) (layer "F.Cu") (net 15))
 (segment (start 18.0 8.0) (end 13.75 7.5) (width 0.15) (layer "F.Cu") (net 15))
 (segment (start 9.5 12.0) (end 4.5 13.0) (width 0.15) (layer "F.Cu") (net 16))
 (segment (start 12.6 15.5) (end 12.6 23.5) (width 0.15) (layer "F.Cu") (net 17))
 (segment (start 12.2 15.5) (end 12.2 23.5) (width 0.15) (layer "F.Cu") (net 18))
 (segment (start 9.5 22.5) (end 11.4 23.5) (width 0.15) (layer "F.Cu") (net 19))
 (segment (start 16.5 22.5) (end 14.6 23.5) (width 0.15) (layer "F.Cu") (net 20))
 (segment (start 4.4 19.0) (end 3.5 17.0) (width 0.15) (layer "F.Cu") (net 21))
 (via (at 6.0 6.0) (size 0.45) (drill 0.2) (layers "F.Cu" "B.Cu") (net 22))
 (via (at 13.0 12.0) (size 0.45) (drill 0.2) (layers "F.Cu" "B.Cu") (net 22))
 (via (at 20.0 5.0) (size 0.45) (drill 0.2) (layers "F.Cu" "B.Cu") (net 22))
 (via (at 6.0 16.0) (size 0.45) (drill 0.2) (layers "F.Cu" "B.Cu") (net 22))
 (via (at 20.0 20.0) (size 0.45) (drill 0.2) (layers "F.Cu" "B.Cu") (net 22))
 (via (at 13.0 9.0) (size 0.45) (drill 0.2) (layers "F.Cu" "B.Cu") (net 22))
 (via (at 13.0 17.0) (size 0.45) (drill 0.2) (layers "F.Cu" "B.Cu") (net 22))
 (via (at 4.0 13.0) (size 0.45) (drill 0.2) (layers "F.Cu" "B.Cu") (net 22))
 (via (at 22.0 13.0) (size 0.45) (drill 0.2) (layers "F.Cu" "B.Cu") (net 22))
 (via (at 13.0 21.0) (size 0.45) (drill 0.2) (layers "F.Cu" "B.Cu") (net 22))
 (via (at 10.0 14.0) (size 0.45) (drill 0.2) (layers "F.Cu" "B.Cu") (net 22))
 (via (at 16.0 14.0) (size 0.45) (drill 0.2) (layers "F.Cu" "B.Cu") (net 22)))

